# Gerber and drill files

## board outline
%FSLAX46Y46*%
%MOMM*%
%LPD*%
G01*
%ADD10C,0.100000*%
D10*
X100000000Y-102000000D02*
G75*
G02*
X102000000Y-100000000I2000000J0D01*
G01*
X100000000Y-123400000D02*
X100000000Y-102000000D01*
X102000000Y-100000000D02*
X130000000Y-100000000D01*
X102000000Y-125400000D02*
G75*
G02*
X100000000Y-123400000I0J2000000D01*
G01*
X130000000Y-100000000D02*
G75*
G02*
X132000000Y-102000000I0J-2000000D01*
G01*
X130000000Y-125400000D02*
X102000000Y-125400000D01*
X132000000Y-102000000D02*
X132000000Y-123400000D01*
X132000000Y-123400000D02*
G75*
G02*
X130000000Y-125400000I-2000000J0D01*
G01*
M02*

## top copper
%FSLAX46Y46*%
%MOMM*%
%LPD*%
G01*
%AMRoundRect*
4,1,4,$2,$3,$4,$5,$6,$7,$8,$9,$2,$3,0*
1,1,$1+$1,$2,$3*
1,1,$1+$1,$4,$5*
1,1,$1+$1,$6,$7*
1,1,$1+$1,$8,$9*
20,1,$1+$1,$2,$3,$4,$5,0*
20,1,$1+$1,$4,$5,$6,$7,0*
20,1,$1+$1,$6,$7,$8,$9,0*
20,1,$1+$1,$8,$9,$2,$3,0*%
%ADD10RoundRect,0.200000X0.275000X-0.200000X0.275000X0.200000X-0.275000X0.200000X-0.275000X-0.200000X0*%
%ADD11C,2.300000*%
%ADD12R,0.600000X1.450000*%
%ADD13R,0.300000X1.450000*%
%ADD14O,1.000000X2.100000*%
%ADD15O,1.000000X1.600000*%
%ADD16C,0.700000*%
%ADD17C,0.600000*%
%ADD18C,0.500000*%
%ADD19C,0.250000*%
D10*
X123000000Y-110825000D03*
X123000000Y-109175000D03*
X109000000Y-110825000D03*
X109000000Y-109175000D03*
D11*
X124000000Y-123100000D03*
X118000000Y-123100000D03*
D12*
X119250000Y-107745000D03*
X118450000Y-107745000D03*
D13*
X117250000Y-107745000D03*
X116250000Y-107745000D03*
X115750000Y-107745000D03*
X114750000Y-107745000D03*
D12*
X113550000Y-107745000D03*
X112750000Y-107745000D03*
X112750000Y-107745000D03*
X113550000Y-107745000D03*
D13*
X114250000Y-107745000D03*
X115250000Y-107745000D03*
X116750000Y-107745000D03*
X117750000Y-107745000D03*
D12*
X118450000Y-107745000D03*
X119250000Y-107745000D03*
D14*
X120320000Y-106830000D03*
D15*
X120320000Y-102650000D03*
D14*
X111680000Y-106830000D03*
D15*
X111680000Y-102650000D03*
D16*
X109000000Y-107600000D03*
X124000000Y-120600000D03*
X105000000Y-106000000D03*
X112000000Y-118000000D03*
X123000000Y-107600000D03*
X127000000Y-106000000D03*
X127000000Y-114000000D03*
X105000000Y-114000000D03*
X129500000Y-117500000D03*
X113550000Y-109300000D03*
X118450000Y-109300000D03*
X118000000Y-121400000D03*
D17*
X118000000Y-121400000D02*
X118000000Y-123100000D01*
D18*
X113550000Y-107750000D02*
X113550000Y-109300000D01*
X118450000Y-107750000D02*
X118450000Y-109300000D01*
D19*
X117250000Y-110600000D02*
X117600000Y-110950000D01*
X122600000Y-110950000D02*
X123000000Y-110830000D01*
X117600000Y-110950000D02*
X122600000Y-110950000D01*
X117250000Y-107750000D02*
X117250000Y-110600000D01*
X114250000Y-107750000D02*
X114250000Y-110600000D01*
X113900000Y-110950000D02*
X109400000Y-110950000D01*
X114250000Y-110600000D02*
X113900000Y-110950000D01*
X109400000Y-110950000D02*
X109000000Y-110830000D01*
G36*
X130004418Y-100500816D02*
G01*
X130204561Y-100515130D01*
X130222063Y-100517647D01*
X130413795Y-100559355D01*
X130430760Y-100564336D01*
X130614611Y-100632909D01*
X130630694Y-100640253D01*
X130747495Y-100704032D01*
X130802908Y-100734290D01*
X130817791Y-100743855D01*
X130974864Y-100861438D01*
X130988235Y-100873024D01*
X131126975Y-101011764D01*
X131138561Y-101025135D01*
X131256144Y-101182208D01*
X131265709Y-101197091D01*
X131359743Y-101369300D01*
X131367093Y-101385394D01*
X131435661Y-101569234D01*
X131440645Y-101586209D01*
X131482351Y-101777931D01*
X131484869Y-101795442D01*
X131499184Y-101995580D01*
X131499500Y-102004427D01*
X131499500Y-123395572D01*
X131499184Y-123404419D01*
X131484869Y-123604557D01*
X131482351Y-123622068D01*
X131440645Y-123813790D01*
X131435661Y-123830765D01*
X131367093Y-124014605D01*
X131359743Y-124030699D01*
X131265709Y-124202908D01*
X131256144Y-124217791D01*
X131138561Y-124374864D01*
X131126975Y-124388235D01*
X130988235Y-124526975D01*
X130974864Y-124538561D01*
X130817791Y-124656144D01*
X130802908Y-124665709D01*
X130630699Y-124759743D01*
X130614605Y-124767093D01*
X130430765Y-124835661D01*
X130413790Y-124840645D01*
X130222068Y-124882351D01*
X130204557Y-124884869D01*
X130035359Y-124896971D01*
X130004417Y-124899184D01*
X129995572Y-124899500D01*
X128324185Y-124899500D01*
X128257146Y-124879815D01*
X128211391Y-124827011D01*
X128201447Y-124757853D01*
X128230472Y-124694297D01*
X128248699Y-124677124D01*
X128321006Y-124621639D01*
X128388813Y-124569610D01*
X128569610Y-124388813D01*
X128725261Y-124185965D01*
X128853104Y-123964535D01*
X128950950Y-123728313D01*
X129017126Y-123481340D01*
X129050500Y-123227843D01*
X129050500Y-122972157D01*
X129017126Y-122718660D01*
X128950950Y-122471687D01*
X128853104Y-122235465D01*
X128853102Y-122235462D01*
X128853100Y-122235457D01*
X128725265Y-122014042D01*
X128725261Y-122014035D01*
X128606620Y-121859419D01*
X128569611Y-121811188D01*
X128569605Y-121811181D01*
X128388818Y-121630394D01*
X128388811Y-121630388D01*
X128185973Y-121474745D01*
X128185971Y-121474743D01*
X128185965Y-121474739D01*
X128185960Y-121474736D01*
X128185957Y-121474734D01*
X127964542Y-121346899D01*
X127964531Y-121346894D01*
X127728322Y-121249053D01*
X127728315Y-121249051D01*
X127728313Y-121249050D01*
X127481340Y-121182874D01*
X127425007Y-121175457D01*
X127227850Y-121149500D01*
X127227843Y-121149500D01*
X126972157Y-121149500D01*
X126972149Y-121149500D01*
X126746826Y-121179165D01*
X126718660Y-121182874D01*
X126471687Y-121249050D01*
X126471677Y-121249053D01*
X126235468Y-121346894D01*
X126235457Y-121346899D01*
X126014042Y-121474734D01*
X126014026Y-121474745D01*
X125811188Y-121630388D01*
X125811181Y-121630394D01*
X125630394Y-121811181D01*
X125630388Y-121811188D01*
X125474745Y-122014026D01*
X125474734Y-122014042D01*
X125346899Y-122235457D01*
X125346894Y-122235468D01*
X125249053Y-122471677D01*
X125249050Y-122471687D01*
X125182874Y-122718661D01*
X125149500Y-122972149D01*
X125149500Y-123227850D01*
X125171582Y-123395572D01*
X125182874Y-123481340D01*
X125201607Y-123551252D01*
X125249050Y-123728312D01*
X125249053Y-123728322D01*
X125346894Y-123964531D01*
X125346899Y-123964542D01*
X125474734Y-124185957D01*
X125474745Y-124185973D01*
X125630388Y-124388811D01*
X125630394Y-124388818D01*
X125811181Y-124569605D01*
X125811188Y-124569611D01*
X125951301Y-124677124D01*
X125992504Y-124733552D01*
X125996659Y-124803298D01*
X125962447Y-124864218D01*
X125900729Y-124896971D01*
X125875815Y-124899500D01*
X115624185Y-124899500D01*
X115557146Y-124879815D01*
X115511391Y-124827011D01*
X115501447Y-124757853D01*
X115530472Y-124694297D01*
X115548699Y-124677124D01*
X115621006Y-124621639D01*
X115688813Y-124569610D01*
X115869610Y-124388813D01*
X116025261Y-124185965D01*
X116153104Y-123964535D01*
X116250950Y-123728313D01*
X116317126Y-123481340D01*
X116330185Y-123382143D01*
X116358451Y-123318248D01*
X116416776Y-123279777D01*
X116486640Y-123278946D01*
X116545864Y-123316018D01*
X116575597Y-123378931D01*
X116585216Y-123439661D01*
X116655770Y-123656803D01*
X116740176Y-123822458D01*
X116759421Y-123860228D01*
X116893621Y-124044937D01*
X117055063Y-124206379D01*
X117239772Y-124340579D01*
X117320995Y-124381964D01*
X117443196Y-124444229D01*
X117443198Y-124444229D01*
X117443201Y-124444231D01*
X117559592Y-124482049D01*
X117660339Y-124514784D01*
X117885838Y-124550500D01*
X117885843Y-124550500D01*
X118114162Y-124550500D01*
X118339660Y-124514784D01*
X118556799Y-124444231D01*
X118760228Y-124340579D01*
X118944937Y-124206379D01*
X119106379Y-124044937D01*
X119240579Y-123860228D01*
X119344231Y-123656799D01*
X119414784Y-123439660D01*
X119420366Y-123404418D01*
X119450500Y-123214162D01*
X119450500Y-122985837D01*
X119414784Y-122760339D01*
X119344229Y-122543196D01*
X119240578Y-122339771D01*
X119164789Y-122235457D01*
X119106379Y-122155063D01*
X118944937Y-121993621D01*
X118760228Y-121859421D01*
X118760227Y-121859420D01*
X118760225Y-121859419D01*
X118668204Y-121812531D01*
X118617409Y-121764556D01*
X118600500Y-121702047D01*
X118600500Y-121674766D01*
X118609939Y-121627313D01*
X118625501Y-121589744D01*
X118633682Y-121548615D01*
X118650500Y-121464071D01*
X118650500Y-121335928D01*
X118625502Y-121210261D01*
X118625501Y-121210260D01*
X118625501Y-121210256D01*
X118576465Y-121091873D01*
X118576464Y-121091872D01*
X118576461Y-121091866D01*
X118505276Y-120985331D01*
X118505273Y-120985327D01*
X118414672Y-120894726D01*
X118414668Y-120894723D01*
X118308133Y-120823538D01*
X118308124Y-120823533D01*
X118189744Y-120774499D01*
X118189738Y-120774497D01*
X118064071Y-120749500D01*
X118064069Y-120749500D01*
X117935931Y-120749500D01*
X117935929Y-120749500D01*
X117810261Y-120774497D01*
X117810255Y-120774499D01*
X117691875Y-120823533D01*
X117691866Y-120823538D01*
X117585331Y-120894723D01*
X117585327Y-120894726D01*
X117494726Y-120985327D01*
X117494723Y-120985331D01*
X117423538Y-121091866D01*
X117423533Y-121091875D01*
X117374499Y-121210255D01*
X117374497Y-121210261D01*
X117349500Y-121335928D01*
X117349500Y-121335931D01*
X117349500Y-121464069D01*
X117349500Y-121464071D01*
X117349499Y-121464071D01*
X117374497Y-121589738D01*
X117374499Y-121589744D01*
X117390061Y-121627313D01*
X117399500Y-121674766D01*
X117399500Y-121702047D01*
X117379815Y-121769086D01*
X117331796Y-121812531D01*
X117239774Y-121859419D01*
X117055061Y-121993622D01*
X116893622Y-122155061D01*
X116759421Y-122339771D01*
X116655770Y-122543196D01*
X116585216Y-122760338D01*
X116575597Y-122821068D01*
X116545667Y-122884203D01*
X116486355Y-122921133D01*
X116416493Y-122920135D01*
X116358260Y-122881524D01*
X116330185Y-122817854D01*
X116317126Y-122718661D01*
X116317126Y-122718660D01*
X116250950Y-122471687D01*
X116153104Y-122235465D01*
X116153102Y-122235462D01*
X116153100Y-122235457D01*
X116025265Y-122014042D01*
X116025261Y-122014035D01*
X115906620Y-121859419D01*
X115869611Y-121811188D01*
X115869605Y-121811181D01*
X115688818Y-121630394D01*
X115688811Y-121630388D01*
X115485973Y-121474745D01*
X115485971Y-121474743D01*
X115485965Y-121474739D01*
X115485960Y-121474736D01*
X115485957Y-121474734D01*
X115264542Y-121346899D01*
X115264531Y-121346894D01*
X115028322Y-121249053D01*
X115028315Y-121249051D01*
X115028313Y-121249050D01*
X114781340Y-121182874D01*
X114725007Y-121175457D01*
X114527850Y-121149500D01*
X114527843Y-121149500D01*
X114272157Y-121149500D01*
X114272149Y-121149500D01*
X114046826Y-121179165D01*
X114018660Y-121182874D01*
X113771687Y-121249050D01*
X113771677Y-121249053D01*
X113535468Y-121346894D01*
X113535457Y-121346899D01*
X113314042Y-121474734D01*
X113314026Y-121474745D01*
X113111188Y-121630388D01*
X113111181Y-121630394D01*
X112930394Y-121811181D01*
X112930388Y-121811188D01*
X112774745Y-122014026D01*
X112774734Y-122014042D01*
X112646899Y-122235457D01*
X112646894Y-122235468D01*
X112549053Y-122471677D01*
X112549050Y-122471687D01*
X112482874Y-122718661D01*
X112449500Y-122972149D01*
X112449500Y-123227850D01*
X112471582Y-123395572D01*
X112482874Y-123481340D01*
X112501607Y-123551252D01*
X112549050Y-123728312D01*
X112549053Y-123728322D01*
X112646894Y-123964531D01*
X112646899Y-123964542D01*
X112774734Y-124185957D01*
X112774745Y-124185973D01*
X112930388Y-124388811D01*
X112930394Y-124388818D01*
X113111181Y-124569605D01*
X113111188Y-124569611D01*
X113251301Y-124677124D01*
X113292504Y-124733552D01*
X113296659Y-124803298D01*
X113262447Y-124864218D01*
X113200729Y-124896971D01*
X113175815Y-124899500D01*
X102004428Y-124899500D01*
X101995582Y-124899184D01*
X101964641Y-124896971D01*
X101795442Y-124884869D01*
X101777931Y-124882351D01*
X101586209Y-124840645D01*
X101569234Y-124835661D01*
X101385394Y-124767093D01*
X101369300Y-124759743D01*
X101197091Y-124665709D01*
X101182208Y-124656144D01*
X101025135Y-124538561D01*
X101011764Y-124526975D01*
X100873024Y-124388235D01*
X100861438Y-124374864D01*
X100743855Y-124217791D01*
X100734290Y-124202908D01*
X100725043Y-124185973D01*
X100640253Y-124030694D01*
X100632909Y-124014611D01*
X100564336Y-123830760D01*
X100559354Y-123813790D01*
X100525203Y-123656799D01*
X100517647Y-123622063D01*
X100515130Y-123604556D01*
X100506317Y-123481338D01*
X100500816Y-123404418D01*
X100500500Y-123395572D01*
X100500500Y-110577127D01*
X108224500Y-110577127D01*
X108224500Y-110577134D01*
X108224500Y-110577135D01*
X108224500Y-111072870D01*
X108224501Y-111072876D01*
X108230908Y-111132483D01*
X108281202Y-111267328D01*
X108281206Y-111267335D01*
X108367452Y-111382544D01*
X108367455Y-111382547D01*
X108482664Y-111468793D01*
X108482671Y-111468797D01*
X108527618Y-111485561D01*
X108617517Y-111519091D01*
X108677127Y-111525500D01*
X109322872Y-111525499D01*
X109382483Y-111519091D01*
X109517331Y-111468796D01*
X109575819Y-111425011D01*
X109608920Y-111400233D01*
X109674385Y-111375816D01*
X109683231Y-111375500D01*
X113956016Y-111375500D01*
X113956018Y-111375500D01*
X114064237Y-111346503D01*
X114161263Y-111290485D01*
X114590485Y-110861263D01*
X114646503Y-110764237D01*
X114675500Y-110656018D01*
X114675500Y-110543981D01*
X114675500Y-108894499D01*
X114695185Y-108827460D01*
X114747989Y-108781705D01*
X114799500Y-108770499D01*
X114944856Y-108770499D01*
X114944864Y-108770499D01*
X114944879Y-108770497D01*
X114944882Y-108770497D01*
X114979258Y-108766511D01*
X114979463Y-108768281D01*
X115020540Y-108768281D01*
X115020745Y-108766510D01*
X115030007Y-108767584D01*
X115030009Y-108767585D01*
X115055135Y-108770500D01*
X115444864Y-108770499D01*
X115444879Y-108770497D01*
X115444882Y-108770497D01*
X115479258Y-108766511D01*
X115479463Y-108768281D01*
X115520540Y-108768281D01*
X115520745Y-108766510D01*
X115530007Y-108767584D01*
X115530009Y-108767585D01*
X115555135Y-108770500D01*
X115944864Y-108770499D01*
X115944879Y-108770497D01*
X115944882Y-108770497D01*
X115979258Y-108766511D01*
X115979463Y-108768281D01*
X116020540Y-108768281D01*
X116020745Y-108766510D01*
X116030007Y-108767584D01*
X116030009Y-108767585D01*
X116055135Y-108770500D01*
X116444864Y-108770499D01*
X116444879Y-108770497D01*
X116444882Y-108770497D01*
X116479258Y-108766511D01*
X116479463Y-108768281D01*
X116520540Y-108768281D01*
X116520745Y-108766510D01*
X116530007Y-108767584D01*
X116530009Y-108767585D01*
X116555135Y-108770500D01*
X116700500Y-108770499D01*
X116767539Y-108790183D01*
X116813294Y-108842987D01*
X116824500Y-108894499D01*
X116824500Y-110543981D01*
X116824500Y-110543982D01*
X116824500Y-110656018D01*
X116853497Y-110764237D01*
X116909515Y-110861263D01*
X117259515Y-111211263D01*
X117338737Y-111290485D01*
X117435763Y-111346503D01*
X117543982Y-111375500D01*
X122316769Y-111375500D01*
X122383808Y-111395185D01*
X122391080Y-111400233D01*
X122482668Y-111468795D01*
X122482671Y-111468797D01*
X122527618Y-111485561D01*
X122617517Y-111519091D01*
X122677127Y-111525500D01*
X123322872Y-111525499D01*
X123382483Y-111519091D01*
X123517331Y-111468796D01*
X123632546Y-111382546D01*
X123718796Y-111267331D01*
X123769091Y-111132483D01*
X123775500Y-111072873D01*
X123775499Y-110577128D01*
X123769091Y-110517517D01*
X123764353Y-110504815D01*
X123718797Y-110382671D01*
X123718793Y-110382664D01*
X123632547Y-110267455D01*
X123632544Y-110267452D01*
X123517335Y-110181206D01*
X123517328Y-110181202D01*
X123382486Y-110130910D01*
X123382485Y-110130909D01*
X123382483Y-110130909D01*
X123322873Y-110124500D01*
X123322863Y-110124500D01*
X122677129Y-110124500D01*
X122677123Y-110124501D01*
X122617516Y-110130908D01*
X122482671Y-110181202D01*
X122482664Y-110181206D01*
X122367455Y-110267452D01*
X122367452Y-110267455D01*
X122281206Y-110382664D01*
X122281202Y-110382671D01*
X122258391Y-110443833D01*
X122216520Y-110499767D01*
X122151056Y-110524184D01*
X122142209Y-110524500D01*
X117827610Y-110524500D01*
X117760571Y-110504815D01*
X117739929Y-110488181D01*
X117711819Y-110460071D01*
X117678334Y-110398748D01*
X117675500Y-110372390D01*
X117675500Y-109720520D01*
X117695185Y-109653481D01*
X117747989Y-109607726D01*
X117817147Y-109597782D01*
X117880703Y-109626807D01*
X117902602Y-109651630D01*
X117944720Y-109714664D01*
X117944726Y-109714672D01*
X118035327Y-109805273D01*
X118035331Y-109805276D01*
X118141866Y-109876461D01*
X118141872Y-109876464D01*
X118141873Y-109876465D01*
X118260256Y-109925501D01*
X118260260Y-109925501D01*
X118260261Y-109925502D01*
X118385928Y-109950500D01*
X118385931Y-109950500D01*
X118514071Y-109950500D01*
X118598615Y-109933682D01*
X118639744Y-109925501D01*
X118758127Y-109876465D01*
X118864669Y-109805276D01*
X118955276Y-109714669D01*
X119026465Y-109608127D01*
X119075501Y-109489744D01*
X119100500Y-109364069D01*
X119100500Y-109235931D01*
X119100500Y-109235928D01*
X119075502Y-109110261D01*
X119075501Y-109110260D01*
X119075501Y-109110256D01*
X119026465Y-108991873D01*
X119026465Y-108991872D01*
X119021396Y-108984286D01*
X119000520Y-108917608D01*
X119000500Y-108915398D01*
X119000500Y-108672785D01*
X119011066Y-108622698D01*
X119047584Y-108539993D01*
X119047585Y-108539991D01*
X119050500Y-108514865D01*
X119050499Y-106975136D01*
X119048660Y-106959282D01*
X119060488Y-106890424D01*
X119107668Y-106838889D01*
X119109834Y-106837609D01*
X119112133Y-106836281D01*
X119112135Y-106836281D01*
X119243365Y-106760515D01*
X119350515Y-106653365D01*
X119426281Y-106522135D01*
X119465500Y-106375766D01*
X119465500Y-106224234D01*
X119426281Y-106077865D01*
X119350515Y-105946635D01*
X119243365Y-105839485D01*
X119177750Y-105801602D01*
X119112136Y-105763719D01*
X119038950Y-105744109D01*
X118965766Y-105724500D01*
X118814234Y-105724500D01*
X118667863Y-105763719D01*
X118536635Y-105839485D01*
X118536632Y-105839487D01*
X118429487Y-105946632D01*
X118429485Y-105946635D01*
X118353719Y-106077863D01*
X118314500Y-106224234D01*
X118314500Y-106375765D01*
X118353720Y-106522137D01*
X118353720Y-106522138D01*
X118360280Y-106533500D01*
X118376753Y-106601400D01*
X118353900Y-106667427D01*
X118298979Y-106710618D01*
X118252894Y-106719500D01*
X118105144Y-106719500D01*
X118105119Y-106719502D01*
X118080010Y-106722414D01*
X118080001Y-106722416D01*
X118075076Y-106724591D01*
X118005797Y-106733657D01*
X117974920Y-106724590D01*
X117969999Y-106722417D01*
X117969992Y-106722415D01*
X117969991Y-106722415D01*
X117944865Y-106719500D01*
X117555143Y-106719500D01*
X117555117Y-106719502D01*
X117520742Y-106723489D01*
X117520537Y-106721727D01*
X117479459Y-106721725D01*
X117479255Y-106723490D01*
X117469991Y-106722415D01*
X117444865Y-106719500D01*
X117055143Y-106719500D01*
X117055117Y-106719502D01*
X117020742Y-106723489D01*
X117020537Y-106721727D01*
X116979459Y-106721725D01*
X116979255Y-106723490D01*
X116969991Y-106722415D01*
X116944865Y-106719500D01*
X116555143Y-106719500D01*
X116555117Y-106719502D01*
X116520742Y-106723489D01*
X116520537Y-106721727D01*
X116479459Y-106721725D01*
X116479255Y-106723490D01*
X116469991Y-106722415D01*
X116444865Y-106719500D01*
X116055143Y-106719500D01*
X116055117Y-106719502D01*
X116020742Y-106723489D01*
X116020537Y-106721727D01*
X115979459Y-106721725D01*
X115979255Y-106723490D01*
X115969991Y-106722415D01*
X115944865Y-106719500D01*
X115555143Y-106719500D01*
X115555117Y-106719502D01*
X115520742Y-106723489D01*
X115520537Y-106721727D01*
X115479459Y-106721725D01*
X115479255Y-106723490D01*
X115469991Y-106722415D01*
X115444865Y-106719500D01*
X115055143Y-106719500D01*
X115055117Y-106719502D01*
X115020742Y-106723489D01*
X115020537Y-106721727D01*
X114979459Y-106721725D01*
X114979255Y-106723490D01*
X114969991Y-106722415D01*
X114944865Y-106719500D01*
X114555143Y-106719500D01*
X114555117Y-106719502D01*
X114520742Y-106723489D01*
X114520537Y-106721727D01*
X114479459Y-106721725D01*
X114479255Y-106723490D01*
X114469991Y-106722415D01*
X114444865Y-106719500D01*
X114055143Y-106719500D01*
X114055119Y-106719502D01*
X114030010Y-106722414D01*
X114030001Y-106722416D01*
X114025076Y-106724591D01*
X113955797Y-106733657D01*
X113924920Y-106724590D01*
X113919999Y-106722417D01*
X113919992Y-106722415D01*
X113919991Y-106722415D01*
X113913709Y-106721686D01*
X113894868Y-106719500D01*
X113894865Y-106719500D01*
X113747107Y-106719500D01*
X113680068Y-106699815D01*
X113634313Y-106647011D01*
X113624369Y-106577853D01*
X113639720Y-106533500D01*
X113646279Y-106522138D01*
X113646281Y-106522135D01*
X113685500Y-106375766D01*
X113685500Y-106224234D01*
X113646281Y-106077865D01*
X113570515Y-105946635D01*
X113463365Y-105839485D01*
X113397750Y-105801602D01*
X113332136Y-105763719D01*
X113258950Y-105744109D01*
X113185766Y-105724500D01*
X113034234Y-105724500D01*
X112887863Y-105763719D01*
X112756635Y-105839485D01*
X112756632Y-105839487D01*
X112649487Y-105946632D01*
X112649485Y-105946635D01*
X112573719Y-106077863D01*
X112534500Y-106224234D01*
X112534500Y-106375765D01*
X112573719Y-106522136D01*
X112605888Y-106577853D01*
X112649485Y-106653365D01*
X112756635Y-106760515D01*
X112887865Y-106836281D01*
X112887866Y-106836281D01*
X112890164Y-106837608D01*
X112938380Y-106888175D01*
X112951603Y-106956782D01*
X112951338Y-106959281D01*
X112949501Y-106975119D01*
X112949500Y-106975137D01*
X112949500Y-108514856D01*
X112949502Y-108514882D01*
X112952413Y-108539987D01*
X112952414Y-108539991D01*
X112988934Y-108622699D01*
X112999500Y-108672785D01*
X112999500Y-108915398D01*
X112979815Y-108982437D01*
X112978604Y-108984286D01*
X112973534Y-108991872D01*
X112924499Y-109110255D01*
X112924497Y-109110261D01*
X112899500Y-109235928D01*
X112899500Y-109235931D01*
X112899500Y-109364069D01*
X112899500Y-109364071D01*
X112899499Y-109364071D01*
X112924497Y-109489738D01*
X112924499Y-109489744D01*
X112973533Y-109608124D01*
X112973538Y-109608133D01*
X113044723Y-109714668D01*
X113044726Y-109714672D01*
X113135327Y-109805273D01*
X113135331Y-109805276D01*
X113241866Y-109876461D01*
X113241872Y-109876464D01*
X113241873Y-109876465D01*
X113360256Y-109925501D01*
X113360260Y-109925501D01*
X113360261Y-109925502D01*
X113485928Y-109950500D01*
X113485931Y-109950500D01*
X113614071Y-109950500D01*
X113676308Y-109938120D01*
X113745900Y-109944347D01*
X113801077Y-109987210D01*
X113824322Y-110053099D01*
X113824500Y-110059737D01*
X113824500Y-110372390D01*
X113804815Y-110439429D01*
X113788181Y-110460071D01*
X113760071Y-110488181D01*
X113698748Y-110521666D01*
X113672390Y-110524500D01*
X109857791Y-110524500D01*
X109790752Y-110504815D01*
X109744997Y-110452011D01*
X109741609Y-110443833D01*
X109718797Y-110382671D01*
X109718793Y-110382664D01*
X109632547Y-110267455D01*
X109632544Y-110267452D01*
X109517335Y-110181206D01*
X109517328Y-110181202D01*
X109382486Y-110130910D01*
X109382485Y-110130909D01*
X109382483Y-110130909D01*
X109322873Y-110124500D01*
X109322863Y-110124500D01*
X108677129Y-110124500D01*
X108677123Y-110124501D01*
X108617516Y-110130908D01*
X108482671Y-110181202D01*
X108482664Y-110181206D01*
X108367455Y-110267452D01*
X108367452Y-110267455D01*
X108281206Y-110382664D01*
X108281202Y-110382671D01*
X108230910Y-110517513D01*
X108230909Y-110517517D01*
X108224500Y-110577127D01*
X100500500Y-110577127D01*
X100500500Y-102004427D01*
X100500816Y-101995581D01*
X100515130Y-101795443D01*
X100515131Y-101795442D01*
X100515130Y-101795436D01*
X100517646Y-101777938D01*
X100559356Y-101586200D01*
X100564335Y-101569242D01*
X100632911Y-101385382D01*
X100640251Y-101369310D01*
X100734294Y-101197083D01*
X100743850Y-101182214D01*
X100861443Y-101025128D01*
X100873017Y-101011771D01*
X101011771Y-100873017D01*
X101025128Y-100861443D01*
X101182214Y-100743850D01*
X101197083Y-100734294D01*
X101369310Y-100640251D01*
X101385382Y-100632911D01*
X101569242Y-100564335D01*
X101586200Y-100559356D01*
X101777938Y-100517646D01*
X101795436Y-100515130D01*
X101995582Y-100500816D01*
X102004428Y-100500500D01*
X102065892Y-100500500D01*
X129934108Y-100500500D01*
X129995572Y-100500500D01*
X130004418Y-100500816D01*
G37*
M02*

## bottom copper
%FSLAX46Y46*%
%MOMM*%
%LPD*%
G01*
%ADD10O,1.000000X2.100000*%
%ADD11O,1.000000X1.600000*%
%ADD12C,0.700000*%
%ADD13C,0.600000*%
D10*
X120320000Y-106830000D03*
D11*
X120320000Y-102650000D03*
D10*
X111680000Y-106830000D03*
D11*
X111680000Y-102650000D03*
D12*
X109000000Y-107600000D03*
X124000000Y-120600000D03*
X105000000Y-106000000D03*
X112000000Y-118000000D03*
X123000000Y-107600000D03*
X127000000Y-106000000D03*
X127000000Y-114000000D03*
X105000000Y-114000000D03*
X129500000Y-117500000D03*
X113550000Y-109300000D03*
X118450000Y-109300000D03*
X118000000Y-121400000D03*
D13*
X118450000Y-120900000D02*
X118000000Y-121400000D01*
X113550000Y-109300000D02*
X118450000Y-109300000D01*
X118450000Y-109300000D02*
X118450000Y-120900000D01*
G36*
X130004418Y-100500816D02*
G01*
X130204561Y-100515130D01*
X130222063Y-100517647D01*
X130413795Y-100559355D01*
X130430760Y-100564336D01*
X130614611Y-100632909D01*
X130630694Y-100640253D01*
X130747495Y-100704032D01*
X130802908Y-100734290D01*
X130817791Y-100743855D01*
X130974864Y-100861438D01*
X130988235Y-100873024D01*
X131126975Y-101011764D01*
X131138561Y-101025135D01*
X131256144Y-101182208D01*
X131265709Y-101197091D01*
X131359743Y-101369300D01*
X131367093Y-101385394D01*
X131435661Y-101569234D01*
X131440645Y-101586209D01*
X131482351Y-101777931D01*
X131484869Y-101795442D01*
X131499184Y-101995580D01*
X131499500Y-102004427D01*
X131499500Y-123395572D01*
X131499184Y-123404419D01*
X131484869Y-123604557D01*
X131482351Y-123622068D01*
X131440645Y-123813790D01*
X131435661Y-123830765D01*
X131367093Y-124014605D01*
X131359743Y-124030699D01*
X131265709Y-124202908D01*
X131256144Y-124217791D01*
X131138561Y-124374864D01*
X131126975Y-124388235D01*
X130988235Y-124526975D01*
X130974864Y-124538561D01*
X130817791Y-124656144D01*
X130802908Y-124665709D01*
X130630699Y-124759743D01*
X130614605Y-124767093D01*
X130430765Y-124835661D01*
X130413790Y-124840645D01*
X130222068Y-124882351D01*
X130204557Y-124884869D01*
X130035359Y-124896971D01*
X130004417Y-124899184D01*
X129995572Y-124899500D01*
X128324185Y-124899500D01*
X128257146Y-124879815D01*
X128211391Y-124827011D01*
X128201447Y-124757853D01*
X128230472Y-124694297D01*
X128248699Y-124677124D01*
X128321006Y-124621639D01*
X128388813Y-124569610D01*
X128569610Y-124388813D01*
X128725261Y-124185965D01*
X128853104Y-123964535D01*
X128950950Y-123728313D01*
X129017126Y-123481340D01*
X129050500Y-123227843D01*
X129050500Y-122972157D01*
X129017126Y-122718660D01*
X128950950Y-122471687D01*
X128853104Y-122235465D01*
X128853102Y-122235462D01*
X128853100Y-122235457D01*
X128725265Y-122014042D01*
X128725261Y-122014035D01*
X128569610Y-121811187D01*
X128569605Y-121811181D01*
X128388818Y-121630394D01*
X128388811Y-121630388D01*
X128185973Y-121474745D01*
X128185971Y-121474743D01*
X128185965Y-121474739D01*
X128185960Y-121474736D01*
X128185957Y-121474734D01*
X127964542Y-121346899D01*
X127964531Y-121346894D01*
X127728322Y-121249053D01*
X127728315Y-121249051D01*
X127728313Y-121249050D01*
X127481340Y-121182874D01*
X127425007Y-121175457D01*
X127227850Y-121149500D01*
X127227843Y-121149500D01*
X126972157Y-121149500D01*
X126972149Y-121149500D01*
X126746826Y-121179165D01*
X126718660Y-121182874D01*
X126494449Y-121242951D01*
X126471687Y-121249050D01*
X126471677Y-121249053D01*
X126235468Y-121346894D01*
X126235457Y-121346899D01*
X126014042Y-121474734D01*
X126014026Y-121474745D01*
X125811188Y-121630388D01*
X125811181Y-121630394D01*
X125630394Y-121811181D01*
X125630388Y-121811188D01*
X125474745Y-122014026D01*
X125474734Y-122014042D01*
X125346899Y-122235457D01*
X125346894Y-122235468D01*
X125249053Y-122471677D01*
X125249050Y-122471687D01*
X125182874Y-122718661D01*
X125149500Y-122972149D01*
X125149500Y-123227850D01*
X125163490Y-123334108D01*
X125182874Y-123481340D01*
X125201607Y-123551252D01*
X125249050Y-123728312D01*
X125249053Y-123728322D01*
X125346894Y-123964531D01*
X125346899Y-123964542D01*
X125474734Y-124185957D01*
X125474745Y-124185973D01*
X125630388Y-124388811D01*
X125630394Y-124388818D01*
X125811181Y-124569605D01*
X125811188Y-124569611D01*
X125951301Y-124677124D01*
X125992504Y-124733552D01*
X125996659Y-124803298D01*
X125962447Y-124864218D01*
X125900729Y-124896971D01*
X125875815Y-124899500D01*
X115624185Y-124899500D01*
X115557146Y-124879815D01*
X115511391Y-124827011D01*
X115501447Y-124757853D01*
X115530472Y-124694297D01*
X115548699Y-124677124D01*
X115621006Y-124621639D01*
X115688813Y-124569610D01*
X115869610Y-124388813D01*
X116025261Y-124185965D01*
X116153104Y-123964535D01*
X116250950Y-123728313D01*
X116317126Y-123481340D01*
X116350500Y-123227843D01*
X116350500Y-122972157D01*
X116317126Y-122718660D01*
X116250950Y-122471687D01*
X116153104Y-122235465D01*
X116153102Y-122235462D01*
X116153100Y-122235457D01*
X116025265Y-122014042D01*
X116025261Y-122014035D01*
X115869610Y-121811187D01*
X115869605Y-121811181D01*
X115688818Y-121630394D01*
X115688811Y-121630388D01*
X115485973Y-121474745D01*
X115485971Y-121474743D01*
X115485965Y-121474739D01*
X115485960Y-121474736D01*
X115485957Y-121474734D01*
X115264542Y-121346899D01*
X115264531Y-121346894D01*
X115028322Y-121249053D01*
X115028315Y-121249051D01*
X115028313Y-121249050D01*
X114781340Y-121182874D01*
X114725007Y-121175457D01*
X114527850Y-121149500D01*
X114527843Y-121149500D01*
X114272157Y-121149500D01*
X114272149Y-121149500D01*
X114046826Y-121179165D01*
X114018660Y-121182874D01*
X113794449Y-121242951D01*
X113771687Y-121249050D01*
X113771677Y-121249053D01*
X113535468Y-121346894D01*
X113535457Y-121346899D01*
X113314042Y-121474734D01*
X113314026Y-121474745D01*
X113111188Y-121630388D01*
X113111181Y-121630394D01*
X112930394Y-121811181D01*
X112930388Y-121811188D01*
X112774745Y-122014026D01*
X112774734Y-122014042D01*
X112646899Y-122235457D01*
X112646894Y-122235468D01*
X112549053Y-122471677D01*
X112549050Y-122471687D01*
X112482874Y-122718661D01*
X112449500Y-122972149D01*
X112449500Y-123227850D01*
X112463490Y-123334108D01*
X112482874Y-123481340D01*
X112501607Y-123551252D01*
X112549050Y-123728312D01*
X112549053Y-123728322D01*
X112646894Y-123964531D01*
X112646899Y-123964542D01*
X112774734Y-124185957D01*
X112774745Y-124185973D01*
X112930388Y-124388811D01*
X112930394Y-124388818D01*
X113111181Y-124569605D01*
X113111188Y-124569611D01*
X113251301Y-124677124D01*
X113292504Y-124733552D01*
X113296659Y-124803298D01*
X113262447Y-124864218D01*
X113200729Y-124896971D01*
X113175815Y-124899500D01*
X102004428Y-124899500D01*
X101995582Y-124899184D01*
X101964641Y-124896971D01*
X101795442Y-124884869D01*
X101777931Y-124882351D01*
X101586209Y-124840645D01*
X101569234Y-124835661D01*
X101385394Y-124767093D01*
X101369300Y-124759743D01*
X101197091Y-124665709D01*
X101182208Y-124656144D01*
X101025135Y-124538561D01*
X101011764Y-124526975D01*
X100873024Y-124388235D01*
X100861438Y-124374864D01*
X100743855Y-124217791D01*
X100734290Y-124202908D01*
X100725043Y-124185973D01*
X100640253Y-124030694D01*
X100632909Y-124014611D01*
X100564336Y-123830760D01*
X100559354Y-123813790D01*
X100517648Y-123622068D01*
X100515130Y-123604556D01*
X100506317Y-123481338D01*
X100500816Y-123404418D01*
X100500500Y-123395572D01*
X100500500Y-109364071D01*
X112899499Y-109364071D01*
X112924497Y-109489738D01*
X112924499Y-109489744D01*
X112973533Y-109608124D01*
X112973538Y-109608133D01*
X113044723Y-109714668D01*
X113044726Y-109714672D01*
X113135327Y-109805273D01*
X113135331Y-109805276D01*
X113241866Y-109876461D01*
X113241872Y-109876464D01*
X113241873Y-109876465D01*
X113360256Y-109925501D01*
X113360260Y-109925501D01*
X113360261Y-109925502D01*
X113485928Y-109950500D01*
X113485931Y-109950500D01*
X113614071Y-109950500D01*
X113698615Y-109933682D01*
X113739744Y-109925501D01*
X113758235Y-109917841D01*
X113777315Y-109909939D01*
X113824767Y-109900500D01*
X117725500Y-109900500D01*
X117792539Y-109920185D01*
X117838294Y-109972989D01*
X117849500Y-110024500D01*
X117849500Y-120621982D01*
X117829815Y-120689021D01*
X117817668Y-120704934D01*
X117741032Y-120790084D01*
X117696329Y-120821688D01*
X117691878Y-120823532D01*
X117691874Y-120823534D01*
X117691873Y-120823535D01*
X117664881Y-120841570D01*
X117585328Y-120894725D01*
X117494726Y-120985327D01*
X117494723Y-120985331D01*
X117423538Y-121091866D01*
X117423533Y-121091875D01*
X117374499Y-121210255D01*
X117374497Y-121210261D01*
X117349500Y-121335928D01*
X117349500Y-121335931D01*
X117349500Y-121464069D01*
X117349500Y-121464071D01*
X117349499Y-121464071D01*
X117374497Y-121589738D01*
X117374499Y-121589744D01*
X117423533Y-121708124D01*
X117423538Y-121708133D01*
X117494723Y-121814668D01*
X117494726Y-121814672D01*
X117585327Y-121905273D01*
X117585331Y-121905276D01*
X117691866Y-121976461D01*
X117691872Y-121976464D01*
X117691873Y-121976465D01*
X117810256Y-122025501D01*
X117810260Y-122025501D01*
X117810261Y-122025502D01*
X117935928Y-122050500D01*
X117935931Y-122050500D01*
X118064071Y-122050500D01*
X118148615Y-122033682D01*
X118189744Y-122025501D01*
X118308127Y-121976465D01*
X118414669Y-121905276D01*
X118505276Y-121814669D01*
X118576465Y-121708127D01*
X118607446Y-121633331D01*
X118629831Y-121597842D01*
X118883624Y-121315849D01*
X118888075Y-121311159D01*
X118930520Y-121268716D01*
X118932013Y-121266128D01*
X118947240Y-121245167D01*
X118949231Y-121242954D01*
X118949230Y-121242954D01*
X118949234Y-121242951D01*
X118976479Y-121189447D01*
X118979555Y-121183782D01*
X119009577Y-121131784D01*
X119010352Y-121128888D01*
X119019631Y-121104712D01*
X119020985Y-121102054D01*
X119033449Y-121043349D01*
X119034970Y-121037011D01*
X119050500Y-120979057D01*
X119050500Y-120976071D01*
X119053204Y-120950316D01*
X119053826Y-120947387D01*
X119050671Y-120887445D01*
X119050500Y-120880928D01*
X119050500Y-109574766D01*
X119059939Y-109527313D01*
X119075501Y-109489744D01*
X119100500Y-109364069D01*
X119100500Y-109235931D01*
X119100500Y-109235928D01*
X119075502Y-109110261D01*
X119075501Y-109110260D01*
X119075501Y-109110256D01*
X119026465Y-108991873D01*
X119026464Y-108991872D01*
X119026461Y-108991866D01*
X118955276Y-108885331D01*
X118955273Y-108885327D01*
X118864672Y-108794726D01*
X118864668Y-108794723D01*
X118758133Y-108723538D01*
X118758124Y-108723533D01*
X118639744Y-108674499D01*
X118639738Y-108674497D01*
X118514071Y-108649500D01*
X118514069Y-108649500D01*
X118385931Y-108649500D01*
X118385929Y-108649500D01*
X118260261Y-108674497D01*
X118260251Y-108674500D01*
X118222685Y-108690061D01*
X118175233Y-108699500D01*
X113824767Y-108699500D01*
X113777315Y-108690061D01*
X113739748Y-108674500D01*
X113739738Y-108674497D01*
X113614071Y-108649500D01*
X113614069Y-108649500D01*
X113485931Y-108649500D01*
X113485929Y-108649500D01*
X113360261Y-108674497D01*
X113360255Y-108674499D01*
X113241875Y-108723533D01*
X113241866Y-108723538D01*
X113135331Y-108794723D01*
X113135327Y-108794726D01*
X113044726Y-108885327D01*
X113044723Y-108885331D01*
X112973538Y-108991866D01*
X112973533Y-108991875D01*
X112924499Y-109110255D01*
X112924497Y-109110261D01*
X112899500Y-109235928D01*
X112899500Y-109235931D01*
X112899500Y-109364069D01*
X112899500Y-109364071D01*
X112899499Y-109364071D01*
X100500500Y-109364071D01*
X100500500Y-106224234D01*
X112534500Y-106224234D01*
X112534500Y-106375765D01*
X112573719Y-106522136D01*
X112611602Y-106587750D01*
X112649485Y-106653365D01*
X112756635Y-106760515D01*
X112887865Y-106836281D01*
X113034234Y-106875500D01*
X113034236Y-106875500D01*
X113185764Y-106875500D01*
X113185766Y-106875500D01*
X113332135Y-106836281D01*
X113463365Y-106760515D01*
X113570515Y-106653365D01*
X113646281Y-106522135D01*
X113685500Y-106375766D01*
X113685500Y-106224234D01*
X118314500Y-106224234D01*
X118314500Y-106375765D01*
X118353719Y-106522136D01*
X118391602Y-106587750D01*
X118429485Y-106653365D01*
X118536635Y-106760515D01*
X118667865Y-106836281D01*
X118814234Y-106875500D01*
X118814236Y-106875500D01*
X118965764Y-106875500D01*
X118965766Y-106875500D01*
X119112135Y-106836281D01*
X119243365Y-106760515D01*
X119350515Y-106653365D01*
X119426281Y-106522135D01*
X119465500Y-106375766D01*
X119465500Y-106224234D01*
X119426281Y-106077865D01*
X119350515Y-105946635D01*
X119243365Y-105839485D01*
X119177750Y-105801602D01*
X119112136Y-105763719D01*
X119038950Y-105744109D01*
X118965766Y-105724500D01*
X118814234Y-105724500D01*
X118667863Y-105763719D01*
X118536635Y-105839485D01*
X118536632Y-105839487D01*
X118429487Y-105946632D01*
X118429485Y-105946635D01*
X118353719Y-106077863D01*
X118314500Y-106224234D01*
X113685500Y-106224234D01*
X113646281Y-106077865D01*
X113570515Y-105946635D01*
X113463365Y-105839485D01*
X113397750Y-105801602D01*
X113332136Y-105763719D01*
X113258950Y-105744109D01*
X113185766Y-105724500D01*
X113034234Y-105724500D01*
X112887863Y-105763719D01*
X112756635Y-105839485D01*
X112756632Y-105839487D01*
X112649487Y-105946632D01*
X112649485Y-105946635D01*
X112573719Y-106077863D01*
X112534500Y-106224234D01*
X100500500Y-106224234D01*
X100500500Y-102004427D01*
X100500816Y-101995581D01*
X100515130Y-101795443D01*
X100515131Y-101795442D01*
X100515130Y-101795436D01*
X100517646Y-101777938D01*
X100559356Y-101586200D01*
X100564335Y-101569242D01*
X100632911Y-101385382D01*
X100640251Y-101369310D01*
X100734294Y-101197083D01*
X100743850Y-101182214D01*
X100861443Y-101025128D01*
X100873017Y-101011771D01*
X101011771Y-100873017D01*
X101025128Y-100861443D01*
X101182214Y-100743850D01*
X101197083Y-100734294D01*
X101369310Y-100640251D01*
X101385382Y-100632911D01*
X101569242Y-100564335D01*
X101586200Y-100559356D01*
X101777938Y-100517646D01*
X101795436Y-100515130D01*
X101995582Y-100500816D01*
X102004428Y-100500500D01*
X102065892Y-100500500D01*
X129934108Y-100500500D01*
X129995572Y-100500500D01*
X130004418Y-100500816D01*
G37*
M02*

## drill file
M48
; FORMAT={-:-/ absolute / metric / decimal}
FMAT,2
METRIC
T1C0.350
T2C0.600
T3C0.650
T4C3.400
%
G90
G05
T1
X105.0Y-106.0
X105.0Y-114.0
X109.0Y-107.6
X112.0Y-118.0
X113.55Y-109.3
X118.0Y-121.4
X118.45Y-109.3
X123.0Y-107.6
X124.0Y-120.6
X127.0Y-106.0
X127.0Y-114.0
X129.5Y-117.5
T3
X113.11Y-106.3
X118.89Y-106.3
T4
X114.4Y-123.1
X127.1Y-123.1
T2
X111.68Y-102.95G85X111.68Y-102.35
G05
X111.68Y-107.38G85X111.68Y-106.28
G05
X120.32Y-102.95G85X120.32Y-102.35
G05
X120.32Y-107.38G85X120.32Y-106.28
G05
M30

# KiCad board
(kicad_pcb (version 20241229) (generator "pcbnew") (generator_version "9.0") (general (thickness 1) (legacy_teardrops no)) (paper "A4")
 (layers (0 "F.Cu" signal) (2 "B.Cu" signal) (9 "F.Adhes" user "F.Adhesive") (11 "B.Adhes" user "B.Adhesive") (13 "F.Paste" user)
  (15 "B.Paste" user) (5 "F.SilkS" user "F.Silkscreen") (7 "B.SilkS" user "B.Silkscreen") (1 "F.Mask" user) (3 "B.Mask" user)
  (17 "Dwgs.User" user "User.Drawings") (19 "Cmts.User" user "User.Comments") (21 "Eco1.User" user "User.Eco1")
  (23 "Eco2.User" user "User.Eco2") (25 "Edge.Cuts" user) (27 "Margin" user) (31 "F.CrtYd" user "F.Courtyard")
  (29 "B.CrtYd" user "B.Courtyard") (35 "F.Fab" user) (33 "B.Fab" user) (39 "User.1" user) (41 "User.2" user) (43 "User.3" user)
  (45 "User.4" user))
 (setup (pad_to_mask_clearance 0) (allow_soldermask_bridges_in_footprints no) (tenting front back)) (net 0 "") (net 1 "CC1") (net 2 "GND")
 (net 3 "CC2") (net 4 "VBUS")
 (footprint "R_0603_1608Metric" (layer "F.Cu") (at 123 110 90)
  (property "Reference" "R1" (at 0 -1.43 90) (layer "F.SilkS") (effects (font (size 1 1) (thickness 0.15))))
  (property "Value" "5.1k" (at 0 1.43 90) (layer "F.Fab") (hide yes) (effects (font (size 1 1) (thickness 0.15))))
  (pad "1" smd roundrect (at -0.825 0 90) (size 0.8 0.95) (layers "F.Cu" "F.Mask" "F.Paste") (roundrect_rratio 0.25) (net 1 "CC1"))
  (pad "2" smd roundrect (at 0.825 0 90) (size 0.8 0.95) (layers "F.Cu" "F.Mask" "F.Paste") (roundrect_rratio 0.25) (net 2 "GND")))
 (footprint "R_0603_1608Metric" (layer "F.Cu") (at 109 110 90)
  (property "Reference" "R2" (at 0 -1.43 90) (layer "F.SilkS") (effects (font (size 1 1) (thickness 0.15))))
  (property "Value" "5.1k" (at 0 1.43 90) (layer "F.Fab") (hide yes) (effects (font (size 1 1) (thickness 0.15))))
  (pad "1" smd roundrect (at -0.825 0 90) (size 0.8 0.95) (layers "F.Cu" "F.Mask" "F.Paste") (roundrect_rratio 0.25) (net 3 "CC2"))
  (pad "2" smd roundrect (at 0.825 0 90) (size 0.8 0.95) (layers "F.Cu" "F.Mask" "F.Paste") (roundrect_rratio 0.25) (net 2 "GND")))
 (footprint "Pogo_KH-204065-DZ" (layer "F.Cu") (at 124 123.1)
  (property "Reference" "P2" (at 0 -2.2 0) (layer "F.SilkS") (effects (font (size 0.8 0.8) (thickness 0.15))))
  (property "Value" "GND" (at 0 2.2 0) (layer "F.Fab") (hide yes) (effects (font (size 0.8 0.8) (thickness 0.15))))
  (pad "1" smd circle (at 0 0) (size 2.3 2.3) (layers "F.Cu" "F.Mask" "F.Paste") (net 2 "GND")))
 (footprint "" (layer "F.Cu") (at 114.4 123.1)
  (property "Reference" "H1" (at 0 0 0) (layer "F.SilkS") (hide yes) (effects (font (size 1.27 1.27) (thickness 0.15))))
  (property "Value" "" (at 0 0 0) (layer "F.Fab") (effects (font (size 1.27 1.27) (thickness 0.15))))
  (pad "" np_thru_hole circle (at 0 0) (size 3.4 3.4) (drill 3.4) (layers "*.Cu" "*.Mask")))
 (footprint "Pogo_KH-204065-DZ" (layer "F.Cu") (at 118 123.1)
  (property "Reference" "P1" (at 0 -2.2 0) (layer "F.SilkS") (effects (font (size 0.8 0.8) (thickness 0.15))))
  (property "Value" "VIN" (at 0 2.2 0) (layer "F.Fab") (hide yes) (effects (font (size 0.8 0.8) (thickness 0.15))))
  (pad "1" smd circle (at 0 0) (size 2.3 2.3) (layers "F.Cu" "F.Mask" "F.Paste") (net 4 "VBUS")))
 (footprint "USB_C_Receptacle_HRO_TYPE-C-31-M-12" (layer "F.Cu") (at 116 103.7 180)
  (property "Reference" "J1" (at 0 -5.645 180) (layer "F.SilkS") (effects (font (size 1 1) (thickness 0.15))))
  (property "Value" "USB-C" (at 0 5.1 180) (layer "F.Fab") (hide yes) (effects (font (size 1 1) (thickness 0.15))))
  (pad "" np_thru_hole circle (at -2.89 -2.6 180) (size 0.65 0.65) (drill 0.65) (layers "*.Cu" "*.Mask"))
  (pad "" np_thru_hole circle (at 2.89 -2.6 180) (size 0.65 0.65) (drill 0.65) (layers "*.Cu" "*.Mask"))
  (pad "A1" smd rect (at -3.25 -4.045 180) (size 0.6 1.45) (layers "F.Cu" "F.Mask" "F.Paste") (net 2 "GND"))
  (pad "A4" smd rect (at -2.45 -4.045 180) (size 0.6 1.45) (layers "F.Cu" "F.Mask" "F.Paste") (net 4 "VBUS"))
  (pad "A5" smd rect (at -1.25 -4.045 180) (size 0.3 1.45) (layers "F.Cu" "F.Mask" "F.Paste") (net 1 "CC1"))
  (pad "A6" smd rect (at -0.25 -4.045 180) (size 0.3 1.45) (layers "F.Cu" "F.Mask" "F.Paste"))
  (pad "A7" smd rect (at 0.25 -4.045 180) (size 0.3 1.45) (layers "F.Cu" "F.Mask" "F.Paste"))
  (pad "A8" smd rect (at 1.25 -4.045 180) (size 0.3 1.45) (layers "F.Cu" "F.Mask" "F.Paste"))
  (pad "A9" smd rect (at 2.45 -4.045 180) (size 0.6 1.45) (layers "F.Cu" "F.Mask" "F.Paste") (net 4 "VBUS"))
  (pad "A12" smd rect (at 3.25 -4.045 180) (size 0.6 1.45) (layers "F.Cu" "F.Mask" "F.Paste") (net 2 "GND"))
  (pad "B1" smd rect (at 3.25 -4.045 180) (size 0.6 1.45) (layers "F.Cu" "F.Mask" "F.Paste") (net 2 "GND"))
  (pad "B4" smd rect (at 2.45 -4.045 180) (size 0.6 1.45) (layers "F.Cu" "F.Mask" "F.Paste") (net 4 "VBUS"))
  (pad "B5" smd rect (at 1.75 -4.045 180) (size 0.3 1.45) (layers "F.Cu" "F.Mask" "F.Paste") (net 3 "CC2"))
  (pad "B6" smd rect (at 0.75 -4.045 180) (size 0.3 1.45) (layers "F.Cu" "F.Mask" "F.Paste"))
  (pad "B7" smd rect (at -0.75 -4.045 180) (size 0.3 1.45) (layers "F.Cu" "F.Mask" "F.Paste"))
  (pad "B8" smd rect (at -1.75 -4.045 180) (size 0.3 1.45) (layers "F.Cu" "F.Mask" "F.Paste"))
  (pad "B9" smd rect (at -2.45 -4.045 180) (size 0.6 1.45) (layers "F.Cu" "F.Mask" "F.Paste") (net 4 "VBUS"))
  (pad "B12" smd rect (at -3.25 -4.045 180) (size 0.6 1.45) (layers "F.Cu" "F.Mask" "F.Paste") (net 2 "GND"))
  (pad "S1" thru_hole oval (at -4.32 -3.13 180) (size 1 2.1) (drill oval 0.6 1.7) (layers "*.Cu" "*.Mask") (remove_unused_layers no)
   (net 2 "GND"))
  (pad "S1" thru_hole oval (at -4.32 1.05 180) (size 1 1.6) (drill oval 0.6 1.2) (layers "*.Cu" "*.Mask") (remove_unused_layers no)
   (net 2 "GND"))
  (pad "S1" thru_hole oval (at 4.32 -3.13 180) (size 1 2.1) (drill oval 0.6 1.7) (layers "*.Cu" "*.Mask") (remove_unused_layers no)
   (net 2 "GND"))
  (pad "S1" thru_hole oval (at 4.32 1.05 180) (size 1 1.6) (drill oval 0.6 1.2) (layers "*.Cu" "*.Mask") (remove_unused_layers no)
   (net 2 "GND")))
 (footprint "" (layer "F.Cu") (at 127.1 123.1)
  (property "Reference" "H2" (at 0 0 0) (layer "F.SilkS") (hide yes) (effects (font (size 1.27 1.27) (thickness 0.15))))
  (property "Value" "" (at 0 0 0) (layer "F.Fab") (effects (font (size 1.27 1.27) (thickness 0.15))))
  (pad "" np_thru_hole circle (at 0 0) (size 3.4 3.4) (drill 3.4) (layers "*.Cu" "*.Mask")))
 (gr_arc (start 100 102) (mid 100.585786 100.585786) (end 102 100) (stroke (width 0.1) (type default)) (layer "Edge.Cuts"))
 (gr_line (start 100 123.4) (end 100 102) (stroke (width 0.1) (type default)) (layer "Edge.Cuts"))
 (gr_line (start 102 100) (end 130 100) (stroke (width 0.1) (type default)) (layer "Edge.Cuts"))
 (gr_arc (start 102 125.4) (mid 100.585786 124.814214) (end 100 123.4) (stroke (width 0.1) (type default)) (layer "Edge.Cuts"))
 (gr_arc (start 130 100) (mid 131.414214 100.585786) (end 132 102) (stroke (width 0.1) (type default)) (layer "Edge.Cuts"))
 (gr_line (start 130 125.4) (end 102 125.4) (stroke (width 0.1) (type default)) (layer "Edge.Cuts"))
 (gr_line (start 132 102) (end 132 123.4) (stroke (width 0.1) (type default)) (layer "Edge.Cuts"))
 (gr_arc (start 132 123.4) (mid 131.414214 124.814214) (end 130 125.4) (stroke (width 0.1) (type default)) (layer "Edge.Cuts"))
 (via (at 109 107.6) (size 0.7) (drill 0.35) (layers "F.Cu" "B.Cu") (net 2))
 (via (at 124 120.6) (size 0.7) (drill 0.35) (layers "F.Cu" "B.Cu") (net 2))
 (via (at 105 106) (size 0.7) (drill 0.35) (layers "F.Cu" "B.Cu") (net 2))
 (via (at 112 118) (size 0.7) (drill 0.35) (layers "F.Cu" "B.Cu") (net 2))
 (via (at 123 107.6) (size 0.7) (drill 0.35) (layers "F.Cu" "B.Cu") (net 2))
 (via (at 127 106) (size 0.7) (drill 0.35) (layers "F.Cu" "B.Cu") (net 2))
 (via (at 127 114) (size 0.7) (drill 0.35) (layers "F.Cu" "B.Cu") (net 2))
 (via (at 105 114) (size 0.7) (drill 0.35) (layers "F.Cu" "B.Cu") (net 2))
 (via (at 129.5 117.5) (size 0.7) (drill 0.35) (layers "F.Cu" "B.Cu") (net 2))
 (segment (start 118 121.4) (end 118 123.1) (width 0.6) (layer "F.Cu") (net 4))
 (segment (start 113.55 107.75) (end 113.55 109.3) (width 0.5) (layer "F.Cu") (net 4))
 (segment (start 118.45 107.75) (end 118.45 109.3) (width 0.5) (layer "F.Cu") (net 4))
 (via (at 113.55 109.3) (size 0.7) (drill 0.35) (layers "F.Cu" "B.Cu") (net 4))
 (via (at 118.45 109.3) (size 0.7) (drill 0.35) (layers "F.Cu" "B.Cu") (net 4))
 (via (at 118 121.4) (size 0.7) (drill 0.35) (layers "F.Cu" "B.Cu") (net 4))
 (segment (start 118.45 120.9) (end 118 121.4) (width 0.6) (layer "B.Cu") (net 4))
 (segment (start 113.55 109.3) (end 118.45 109.3) (width 0.6) (layer "B.Cu") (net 4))
 (segment (start 118.45 109.3) (end 118.45 120.9) (width 0.6) (layer "B.Cu") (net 4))
 (segment (start 117.25 110.6) (end 117.6 110.95) (width 0.25) (layer "F.Cu") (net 1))
 (segment (start 122.6 110.95) (end 123 110.83) (width 0.25) (layer "F.Cu") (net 1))
 (segment (start 117.6 110.95) (end 122.6 110.95) (width 0.25) (layer "F.Cu") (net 1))
 (segment (start 117.25 107.75) (end 117.25 110.6) (width 0.25) (layer "F.Cu") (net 1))
 (segment (start 114.25 107.75) (end 114.25 110.6) (width 0.25) (layer "F.Cu") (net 3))
 (segment (start 113.9 110.95) (end 109.4 110.95) (width 0.25) (layer "F.Cu") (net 3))
 (segment (start 114.25 110.6) (end 113.9 110.95) (width 0.25) (layer "F.Cu") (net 3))
 (segment (start 109.4 110.95) (end 109 110.83) (width 0.25) (layer "F.Cu") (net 3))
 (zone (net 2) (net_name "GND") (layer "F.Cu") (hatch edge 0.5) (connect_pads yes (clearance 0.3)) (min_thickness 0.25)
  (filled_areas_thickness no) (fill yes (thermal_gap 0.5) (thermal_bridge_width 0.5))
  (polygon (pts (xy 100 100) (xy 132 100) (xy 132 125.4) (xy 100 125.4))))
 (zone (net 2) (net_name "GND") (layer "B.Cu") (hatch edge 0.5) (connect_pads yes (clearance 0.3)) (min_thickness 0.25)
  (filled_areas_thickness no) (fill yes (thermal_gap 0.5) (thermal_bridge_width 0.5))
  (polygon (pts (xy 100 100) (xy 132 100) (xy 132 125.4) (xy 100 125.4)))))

